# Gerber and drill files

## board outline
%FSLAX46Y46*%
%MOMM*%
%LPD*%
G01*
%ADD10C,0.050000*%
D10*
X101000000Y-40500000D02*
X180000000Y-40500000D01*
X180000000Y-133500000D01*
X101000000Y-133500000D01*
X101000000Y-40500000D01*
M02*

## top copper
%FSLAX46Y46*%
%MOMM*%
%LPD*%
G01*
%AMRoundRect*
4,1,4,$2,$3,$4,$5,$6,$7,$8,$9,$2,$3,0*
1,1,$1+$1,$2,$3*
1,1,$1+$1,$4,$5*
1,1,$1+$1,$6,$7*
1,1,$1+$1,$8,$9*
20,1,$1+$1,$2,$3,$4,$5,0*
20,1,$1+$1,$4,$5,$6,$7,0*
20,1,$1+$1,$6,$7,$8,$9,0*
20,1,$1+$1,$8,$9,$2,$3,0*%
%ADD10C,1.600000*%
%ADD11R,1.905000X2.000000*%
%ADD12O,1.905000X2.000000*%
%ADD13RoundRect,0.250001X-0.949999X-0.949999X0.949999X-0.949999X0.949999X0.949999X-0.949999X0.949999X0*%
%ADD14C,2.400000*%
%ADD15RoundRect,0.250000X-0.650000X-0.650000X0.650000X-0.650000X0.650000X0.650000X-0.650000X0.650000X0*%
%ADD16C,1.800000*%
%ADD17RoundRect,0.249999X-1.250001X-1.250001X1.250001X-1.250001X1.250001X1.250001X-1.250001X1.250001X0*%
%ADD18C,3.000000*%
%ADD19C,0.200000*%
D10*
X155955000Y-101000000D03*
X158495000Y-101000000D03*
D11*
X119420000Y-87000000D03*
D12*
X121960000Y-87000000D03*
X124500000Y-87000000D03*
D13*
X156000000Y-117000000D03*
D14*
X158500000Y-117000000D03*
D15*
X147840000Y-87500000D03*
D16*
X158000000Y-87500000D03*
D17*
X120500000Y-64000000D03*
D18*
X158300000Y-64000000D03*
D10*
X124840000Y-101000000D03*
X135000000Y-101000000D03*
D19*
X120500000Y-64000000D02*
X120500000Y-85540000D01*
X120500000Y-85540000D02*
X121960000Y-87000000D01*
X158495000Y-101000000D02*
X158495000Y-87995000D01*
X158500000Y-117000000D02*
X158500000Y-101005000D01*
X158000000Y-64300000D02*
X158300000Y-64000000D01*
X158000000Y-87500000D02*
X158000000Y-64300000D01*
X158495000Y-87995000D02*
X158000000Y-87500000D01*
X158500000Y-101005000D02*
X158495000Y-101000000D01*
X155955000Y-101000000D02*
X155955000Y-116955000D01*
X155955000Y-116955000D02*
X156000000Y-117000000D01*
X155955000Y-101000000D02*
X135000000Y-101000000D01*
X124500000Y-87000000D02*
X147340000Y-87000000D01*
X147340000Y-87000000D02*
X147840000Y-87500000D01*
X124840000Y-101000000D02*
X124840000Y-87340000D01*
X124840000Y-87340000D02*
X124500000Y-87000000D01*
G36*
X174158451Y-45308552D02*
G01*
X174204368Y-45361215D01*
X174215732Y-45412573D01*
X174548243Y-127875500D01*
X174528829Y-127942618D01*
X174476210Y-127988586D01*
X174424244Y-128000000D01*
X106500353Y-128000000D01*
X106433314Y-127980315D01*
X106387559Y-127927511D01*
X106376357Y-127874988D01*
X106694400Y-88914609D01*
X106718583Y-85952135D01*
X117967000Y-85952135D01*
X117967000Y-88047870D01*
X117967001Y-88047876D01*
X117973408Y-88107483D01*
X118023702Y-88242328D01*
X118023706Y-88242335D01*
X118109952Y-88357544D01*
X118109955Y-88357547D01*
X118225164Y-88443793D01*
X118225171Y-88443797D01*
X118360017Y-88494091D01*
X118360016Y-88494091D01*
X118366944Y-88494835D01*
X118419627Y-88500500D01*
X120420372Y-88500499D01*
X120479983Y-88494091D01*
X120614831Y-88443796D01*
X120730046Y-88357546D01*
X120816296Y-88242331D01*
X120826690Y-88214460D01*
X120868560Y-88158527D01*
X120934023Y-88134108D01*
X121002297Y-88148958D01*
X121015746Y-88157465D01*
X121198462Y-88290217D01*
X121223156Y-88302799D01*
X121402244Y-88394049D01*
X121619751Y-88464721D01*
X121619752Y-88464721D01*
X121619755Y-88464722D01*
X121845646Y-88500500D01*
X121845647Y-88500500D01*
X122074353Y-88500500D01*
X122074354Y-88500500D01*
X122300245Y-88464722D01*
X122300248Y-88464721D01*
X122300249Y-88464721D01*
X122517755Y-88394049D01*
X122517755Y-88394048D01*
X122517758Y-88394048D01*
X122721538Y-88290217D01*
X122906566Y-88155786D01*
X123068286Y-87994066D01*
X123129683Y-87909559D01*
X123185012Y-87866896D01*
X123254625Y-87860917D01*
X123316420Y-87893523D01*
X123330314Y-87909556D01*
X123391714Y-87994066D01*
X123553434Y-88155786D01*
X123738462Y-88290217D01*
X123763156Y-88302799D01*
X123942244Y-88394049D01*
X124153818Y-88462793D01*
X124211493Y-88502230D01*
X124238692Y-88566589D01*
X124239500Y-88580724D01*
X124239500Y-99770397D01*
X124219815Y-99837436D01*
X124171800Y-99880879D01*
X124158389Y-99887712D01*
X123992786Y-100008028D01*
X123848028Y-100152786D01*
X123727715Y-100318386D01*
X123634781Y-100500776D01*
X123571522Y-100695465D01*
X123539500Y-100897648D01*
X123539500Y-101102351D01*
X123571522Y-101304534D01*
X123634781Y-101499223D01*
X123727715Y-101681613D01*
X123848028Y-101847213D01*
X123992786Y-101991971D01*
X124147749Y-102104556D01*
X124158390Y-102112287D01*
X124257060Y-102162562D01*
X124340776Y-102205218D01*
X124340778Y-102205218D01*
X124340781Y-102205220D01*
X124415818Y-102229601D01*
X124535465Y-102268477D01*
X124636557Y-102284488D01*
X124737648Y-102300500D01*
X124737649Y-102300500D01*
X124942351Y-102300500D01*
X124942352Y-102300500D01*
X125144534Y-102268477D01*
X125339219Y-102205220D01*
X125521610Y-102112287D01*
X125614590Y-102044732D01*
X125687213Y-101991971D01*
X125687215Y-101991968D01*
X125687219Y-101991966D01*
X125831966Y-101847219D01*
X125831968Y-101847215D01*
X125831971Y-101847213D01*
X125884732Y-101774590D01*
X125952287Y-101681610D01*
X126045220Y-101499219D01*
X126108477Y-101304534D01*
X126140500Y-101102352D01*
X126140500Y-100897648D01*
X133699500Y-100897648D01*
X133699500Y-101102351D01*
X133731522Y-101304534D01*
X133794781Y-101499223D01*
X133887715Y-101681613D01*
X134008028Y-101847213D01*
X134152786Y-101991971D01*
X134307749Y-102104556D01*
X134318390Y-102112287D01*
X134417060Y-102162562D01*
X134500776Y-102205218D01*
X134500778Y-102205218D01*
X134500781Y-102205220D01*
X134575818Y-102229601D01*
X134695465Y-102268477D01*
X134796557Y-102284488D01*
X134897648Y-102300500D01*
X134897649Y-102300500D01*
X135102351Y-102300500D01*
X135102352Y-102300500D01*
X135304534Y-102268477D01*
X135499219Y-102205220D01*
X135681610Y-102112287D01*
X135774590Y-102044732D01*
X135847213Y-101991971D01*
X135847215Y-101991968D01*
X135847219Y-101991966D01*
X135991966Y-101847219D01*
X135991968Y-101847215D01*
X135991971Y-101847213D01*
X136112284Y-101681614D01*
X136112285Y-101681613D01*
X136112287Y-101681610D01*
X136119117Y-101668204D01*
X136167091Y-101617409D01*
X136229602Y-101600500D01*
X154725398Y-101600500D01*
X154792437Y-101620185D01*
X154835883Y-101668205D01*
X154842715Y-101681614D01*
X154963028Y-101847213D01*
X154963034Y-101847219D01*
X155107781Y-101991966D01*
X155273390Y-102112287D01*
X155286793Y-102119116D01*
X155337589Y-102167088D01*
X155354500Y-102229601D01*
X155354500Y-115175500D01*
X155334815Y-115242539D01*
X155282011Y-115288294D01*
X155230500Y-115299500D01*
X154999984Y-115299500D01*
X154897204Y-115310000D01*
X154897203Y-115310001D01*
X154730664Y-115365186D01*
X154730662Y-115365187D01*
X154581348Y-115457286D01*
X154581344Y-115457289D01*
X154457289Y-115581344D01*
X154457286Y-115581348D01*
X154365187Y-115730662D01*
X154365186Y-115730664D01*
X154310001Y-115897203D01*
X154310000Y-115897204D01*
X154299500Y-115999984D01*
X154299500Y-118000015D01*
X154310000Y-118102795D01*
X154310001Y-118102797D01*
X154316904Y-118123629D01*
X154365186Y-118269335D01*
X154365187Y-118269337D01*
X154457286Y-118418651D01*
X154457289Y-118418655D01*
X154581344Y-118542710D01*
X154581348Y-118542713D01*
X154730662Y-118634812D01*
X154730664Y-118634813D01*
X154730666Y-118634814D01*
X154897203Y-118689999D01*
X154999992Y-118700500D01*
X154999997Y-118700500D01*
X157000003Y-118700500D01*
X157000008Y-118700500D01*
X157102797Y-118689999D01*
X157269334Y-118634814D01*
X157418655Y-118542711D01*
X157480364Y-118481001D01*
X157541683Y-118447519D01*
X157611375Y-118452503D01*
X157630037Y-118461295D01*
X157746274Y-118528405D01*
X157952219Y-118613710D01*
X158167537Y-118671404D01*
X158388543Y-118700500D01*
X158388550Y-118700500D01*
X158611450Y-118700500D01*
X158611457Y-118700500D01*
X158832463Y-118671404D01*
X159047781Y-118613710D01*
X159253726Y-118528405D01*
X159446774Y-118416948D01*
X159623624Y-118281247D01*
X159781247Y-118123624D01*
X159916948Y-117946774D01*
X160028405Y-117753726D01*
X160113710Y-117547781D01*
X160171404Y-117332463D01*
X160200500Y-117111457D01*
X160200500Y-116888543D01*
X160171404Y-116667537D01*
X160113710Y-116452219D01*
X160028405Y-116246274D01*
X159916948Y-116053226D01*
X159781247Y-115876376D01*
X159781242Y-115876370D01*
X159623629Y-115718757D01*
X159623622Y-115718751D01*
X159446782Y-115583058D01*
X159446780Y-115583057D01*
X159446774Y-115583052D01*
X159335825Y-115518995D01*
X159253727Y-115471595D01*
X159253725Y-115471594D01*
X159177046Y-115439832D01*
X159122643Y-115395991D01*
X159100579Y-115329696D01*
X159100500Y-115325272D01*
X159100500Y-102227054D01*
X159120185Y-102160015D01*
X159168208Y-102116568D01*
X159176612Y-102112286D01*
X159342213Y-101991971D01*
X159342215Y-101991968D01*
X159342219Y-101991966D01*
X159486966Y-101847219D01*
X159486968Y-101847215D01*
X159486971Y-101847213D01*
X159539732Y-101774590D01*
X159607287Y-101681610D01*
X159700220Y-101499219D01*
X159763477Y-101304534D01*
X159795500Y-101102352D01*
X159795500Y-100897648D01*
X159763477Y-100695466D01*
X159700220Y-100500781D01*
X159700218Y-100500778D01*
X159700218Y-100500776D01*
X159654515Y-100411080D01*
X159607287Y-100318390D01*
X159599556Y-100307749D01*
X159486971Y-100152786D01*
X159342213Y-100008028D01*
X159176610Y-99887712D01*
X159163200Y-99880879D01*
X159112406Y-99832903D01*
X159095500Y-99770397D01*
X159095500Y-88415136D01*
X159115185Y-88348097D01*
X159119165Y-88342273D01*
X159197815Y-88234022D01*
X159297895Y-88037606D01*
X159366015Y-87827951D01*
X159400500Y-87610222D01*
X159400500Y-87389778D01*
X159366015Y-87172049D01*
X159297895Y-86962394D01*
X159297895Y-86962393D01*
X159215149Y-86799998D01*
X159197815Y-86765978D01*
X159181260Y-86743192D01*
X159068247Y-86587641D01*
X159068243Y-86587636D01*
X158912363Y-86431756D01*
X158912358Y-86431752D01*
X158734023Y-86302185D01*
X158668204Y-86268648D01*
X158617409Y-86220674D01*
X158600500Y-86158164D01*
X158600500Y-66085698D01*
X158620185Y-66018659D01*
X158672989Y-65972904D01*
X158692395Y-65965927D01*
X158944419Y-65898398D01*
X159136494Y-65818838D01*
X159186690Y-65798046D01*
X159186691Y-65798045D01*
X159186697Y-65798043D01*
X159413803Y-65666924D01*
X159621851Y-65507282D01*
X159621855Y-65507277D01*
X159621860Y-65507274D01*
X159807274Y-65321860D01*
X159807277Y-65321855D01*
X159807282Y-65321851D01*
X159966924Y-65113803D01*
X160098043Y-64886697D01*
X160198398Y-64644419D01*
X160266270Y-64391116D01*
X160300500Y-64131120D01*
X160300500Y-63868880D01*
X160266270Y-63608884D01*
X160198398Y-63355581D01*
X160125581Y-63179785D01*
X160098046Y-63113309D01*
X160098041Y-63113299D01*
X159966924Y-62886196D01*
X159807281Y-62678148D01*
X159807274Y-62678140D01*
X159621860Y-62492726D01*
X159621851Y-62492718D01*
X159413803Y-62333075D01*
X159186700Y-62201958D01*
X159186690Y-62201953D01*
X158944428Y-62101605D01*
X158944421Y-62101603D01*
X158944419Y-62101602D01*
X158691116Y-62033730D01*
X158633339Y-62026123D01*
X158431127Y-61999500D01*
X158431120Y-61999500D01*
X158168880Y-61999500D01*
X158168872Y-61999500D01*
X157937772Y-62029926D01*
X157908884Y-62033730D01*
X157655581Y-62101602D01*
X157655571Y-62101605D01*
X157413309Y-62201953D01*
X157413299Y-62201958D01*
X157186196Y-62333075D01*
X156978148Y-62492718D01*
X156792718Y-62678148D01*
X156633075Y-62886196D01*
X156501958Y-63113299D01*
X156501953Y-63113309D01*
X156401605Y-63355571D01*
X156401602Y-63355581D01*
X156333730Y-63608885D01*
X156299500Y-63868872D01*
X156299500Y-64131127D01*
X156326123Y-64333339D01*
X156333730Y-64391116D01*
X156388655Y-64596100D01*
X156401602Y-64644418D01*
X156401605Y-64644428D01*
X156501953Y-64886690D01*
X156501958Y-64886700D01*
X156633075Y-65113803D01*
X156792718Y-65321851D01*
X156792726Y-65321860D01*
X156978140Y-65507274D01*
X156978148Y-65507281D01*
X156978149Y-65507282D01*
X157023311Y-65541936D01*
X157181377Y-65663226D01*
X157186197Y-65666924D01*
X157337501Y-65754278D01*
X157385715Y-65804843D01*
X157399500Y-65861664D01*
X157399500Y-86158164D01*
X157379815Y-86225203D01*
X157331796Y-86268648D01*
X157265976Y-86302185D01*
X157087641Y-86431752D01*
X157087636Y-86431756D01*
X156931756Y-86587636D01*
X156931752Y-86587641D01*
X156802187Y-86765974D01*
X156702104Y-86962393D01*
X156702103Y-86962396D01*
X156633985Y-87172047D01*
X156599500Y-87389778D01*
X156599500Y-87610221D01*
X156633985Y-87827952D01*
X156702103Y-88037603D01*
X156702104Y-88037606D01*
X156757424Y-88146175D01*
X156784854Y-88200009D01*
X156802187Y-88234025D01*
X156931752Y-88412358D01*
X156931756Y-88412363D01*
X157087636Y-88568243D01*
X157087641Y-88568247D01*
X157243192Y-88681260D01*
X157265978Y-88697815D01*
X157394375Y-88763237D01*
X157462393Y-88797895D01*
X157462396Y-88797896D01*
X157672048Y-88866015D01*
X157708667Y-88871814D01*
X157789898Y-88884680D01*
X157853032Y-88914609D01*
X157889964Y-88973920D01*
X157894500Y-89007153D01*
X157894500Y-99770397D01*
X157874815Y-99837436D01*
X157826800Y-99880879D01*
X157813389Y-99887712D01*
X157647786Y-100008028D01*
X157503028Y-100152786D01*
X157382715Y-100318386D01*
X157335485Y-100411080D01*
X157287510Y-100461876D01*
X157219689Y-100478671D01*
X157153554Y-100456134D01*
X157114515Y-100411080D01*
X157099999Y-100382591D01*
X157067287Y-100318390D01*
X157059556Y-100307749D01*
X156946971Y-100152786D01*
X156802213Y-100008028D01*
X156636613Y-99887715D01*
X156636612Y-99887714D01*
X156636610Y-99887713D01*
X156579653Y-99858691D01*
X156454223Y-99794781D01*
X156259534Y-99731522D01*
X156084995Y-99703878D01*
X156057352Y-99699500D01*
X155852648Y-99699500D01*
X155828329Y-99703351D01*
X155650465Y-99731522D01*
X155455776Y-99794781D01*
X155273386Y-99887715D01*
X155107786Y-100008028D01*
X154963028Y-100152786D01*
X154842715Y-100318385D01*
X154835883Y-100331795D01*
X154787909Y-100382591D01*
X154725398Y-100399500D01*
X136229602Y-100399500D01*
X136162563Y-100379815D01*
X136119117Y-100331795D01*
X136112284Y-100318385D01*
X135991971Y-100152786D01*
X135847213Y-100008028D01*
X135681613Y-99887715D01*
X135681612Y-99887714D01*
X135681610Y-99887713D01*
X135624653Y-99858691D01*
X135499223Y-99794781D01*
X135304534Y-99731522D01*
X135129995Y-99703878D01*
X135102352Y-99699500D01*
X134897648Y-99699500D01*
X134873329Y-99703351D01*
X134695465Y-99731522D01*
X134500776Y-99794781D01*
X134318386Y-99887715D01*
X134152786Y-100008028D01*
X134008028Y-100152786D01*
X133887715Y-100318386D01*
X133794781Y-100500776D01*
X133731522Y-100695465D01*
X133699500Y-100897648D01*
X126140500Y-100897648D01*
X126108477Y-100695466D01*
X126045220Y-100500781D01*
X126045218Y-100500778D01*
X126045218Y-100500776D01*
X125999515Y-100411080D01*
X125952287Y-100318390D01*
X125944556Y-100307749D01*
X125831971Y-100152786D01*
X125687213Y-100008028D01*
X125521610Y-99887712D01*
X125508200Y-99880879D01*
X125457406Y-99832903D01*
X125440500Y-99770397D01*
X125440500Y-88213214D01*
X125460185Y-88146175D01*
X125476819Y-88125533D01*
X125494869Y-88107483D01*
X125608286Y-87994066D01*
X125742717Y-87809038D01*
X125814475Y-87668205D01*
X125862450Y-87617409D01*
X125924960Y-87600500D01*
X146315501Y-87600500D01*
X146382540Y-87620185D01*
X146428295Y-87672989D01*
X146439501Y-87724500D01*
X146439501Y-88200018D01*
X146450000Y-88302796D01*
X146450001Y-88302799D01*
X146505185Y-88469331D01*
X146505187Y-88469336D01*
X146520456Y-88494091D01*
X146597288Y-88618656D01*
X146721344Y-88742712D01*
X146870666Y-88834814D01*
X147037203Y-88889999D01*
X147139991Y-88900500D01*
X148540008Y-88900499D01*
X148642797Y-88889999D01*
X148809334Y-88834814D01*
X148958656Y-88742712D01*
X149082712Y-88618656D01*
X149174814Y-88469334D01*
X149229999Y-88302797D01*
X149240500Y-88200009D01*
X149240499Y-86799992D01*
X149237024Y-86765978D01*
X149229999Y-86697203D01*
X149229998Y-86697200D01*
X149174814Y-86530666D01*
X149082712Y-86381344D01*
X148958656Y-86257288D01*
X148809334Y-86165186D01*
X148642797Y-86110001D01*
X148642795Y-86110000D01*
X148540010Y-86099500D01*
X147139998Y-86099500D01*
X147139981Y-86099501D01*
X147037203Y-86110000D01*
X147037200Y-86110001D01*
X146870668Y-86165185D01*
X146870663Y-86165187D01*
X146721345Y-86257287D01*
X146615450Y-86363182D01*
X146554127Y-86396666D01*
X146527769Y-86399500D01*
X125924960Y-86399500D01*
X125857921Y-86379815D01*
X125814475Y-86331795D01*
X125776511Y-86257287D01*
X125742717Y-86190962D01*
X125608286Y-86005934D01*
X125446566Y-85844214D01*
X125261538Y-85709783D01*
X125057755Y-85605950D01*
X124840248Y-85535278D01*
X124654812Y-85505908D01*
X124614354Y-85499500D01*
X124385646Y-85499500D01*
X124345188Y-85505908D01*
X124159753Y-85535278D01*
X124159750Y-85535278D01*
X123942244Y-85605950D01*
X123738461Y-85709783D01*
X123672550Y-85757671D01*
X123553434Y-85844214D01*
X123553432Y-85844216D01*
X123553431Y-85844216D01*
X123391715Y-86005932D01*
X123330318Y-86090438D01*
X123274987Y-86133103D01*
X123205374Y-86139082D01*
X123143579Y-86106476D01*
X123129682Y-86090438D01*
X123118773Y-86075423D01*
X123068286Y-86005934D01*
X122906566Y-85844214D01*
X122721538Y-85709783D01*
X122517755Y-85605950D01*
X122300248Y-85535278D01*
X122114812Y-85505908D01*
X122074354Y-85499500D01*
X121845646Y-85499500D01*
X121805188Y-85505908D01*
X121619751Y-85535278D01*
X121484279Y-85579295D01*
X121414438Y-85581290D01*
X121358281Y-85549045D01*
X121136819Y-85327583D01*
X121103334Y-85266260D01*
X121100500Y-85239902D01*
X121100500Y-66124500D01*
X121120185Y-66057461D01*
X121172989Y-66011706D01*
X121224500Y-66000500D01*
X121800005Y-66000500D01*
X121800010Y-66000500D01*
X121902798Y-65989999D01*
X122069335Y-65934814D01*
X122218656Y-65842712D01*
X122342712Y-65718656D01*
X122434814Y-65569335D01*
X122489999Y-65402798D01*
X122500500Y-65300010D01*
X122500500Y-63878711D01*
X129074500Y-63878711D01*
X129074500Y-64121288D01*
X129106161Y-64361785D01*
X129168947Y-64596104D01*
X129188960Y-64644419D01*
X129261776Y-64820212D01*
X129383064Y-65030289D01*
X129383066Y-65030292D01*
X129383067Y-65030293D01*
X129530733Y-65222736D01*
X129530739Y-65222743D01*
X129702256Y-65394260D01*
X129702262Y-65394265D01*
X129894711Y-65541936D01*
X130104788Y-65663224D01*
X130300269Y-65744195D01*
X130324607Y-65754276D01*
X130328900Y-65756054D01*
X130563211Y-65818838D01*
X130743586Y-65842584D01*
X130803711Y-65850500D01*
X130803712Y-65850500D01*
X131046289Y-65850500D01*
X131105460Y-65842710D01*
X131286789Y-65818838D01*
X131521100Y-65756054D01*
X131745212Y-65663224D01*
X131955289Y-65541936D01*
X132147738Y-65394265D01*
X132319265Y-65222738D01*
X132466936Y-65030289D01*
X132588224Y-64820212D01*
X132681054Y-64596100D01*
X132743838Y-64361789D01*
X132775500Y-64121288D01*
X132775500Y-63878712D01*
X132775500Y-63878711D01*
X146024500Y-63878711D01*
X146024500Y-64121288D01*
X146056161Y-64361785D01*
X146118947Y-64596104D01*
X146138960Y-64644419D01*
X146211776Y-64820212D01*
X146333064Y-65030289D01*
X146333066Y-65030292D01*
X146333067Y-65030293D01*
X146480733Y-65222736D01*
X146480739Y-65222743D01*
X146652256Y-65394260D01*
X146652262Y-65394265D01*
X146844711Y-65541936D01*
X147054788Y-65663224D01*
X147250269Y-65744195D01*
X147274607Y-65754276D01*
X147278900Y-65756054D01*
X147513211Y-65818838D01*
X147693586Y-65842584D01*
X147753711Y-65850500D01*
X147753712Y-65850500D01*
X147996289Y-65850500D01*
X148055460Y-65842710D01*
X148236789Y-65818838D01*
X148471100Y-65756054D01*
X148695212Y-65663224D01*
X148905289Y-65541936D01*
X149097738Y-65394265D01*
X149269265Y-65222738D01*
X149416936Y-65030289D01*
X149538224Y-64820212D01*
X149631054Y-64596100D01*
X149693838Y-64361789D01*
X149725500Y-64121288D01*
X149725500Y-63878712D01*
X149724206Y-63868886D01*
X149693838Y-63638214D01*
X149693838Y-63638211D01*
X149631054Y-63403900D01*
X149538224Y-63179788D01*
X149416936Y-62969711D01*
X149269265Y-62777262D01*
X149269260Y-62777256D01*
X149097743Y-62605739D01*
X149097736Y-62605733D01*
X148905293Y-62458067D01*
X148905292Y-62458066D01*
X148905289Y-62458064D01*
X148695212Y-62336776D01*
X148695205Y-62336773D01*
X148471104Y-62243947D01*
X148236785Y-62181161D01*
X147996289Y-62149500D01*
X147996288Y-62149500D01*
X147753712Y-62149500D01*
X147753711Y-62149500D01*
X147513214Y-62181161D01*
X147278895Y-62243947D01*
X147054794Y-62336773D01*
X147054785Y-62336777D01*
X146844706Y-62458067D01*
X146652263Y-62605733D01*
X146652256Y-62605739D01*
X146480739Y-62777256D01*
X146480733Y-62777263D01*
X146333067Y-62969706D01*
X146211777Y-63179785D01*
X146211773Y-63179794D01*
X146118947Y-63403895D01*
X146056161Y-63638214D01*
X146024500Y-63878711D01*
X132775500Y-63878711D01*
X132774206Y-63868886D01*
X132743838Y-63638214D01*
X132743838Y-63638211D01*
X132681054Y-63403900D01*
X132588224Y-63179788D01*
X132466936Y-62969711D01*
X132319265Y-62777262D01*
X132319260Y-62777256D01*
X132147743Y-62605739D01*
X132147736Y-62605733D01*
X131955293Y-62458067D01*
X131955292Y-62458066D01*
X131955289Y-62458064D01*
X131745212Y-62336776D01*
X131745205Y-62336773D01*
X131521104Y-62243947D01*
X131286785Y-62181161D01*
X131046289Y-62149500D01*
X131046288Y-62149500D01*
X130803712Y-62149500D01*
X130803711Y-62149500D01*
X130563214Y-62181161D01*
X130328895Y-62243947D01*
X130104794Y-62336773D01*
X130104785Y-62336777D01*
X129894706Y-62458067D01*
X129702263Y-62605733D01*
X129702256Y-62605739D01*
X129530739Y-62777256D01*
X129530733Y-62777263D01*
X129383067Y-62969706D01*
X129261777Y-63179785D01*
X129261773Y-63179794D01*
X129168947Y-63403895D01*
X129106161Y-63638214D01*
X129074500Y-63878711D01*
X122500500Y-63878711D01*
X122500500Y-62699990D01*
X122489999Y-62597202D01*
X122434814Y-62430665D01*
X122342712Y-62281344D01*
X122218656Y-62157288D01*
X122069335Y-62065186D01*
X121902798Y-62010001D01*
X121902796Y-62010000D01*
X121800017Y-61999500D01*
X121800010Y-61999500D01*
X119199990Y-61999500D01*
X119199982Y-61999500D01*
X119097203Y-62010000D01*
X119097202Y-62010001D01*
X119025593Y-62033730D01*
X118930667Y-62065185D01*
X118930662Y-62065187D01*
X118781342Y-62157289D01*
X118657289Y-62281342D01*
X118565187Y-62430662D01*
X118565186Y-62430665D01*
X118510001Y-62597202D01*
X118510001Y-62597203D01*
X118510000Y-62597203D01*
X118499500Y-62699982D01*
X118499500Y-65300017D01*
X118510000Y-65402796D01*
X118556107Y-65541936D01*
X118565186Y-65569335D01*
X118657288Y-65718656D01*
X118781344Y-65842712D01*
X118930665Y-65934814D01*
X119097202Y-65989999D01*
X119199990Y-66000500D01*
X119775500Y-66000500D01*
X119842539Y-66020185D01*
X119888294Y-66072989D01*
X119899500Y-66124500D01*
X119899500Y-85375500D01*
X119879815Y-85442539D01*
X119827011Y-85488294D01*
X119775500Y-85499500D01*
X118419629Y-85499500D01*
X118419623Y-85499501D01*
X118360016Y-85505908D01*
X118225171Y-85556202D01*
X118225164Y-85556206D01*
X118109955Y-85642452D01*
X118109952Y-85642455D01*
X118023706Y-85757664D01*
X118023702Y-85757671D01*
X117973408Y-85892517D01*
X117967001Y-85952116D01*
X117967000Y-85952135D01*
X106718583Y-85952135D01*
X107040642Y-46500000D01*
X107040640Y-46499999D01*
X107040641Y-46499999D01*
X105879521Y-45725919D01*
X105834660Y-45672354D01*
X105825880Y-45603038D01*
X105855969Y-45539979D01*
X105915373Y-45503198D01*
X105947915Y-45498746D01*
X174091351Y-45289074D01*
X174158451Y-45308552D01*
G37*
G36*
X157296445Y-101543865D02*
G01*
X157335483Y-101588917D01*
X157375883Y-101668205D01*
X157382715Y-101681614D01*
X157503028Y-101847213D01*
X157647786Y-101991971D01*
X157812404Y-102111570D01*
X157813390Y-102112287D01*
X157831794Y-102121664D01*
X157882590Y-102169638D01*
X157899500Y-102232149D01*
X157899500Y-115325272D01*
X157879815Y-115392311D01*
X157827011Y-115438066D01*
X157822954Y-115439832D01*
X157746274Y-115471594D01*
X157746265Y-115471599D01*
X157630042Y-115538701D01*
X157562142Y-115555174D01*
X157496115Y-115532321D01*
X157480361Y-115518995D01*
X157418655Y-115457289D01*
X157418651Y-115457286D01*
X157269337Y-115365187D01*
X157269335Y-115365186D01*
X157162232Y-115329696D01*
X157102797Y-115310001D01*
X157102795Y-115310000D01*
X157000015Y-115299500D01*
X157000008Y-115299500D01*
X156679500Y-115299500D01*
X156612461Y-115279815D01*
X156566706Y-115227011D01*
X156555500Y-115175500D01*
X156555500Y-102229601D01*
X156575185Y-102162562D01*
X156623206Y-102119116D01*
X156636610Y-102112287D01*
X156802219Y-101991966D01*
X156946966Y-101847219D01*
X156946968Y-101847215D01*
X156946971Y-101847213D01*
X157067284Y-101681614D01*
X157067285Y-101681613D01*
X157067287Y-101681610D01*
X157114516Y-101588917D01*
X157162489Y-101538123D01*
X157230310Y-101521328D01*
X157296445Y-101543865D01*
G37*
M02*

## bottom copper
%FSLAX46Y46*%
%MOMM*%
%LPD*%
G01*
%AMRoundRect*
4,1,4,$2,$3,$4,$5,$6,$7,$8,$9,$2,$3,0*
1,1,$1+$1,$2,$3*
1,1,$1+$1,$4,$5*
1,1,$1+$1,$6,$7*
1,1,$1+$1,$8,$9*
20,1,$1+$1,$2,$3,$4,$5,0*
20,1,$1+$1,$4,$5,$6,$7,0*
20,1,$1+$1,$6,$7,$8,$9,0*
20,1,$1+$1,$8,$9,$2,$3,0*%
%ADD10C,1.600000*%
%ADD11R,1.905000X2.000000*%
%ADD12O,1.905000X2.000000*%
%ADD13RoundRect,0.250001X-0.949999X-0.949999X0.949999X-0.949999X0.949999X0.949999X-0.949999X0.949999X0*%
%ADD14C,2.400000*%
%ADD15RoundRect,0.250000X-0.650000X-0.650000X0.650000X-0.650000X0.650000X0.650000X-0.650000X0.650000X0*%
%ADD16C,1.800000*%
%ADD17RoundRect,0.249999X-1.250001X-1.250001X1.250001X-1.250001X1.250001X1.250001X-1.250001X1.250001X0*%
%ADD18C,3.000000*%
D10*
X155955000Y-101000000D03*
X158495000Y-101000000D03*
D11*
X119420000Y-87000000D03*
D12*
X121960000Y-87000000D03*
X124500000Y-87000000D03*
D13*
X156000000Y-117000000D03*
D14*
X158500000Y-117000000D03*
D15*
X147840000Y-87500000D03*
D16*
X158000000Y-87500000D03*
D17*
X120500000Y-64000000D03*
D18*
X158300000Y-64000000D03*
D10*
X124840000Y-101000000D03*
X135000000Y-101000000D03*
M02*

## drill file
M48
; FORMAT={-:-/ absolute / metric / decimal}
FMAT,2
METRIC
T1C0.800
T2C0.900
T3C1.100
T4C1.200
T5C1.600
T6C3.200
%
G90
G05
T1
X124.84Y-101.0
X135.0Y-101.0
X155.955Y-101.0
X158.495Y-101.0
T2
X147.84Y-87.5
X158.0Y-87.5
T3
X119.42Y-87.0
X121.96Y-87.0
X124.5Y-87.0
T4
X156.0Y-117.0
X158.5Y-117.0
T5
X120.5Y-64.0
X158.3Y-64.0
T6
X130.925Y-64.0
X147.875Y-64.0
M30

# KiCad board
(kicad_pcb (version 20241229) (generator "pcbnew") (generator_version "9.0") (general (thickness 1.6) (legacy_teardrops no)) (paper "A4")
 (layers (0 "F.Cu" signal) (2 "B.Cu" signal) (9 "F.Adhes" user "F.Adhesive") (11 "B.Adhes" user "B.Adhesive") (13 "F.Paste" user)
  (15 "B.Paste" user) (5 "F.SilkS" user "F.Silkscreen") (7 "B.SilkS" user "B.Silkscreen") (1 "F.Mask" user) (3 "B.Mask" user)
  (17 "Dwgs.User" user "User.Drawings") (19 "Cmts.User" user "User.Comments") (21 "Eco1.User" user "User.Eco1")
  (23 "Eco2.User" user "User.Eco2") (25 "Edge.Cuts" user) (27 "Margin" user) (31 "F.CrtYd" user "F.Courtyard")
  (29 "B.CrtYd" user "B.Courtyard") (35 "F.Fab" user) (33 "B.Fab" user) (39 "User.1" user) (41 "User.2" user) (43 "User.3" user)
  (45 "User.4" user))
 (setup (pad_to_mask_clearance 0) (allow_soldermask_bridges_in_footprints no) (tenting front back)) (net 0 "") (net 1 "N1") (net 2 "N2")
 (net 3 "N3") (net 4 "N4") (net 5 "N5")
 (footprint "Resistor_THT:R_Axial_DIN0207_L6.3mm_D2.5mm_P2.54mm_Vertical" (layer "F.Cu") (at 155.955 101)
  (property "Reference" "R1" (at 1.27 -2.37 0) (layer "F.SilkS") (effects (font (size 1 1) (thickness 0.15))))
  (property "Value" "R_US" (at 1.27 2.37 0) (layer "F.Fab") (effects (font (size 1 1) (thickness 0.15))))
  (pad "1" thru_hole circle (at 0 0) (size 1.6 1.6) (drill 0.8) (layers "*.Cu" "*.Mask") (remove_unused_layers no) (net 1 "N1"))
  (pad "2" thru_hole circle (at 2.54 0) (size 1.6 1.6) (drill 0.8) (layers "*.Cu" "*.Mask") (remove_unused_layers no) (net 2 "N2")))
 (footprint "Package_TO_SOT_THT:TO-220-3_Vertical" (layer "F.Cu") (at 119.42 87)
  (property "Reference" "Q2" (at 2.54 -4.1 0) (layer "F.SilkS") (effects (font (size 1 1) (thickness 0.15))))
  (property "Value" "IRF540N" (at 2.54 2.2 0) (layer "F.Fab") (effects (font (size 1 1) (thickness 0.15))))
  (pad "1" thru_hole rect (at 0 0) (size 1.905 2) (drill 1.1) (layers "*.Cu" "*.Mask") (remove_unused_layers no) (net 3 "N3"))
  (pad "2" thru_hole oval (at 2.54 0) (size 1.905 2) (drill 1.1) (layers "*.Cu" "*.Mask") (remove_unused_layers no) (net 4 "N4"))
  (pad "3" thru_hole oval (at 5.08 0) (size 1.905 2) (drill 1.1) (layers "*.Cu" "*.Mask") (remove_unused_layers no) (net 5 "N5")))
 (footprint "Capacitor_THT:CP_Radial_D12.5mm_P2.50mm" (layer "F.Cu") (at 156 117)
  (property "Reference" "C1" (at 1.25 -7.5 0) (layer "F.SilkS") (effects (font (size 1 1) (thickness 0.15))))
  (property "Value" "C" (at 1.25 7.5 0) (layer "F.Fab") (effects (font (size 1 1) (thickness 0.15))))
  (pad "1" thru_hole roundrect (at 0 0) (size 2.4 2.4) (drill 1.2) (layers "*.Cu" "*.Mask") (remove_unused_layers no)
   (roundrect_rratio 0.104167) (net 1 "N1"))
  (pad "2" thru_hole circle (at 2.5 0) (size 2.4 2.4) (drill 1.2) (layers "*.Cu" "*.Mask") (remove_unused_layers no) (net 2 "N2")))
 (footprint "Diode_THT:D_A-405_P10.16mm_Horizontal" (layer "F.Cu") (at 147.84 87.5)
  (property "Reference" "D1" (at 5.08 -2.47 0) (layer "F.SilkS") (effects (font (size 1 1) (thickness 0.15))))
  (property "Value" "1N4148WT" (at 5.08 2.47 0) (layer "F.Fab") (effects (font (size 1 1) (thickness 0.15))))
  (pad "1" thru_hole roundrect (at 0 0) (size 1.8 1.8) (drill 0.9) (layers "*.Cu" "*.Mask") (remove_unused_layers no)
   (roundrect_rratio 0.138889) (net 5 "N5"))
  (pad "2" thru_hole circle (at 10.16 0) (size 1.8 1.8) (drill 0.9) (layers "*.Cu" "*.Mask") (remove_unused_layers no) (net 2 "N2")))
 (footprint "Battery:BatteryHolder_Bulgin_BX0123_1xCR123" (layer "F.Cu") (at 120.5 64)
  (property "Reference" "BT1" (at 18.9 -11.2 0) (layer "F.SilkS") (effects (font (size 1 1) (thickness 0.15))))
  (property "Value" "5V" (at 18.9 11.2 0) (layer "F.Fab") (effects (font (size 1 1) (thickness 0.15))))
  (pad "" np_thru_hole circle (at 10.425 0) (size 3.2 3.2) (drill 3.2) (layers "*.Cu" "*.Mask"))
  (pad "" np_thru_hole circle (at 27.375 0) (size 3.2 3.2) (drill 3.2) (layers "*.Cu" "*.Mask"))
  (pad "1" thru_hole roundrect (at 0 0) (size 3 3) (drill 1.6) (layers "*.Cu" "*.Mask") (remove_unused_layers no)
   (roundrect_rratio 0.083333) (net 4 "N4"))
  (pad "2" thru_hole circle (at 37.8 0) (size 3 3) (drill 1.6) (layers "*.Cu" "*.Mask") (remove_unused_layers no) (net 2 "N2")))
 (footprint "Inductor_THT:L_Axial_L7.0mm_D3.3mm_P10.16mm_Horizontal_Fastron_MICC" (layer "F.Cu") (at 124.84 101)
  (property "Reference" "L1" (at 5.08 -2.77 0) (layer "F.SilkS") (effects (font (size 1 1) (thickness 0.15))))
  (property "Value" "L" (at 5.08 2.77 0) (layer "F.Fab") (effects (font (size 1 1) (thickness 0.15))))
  (pad "1" thru_hole circle (at 0 0) (size 1.6 1.6) (drill 0.8) (layers "*.Cu" "*.Mask") (remove_unused_layers no) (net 5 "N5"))
  (pad "2" thru_hole circle (at 10.16 0) (size 1.6 1.6) (drill 0.8) (layers "*.Cu" "*.Mask") (remove_unused_layers no) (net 1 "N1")))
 (gr_rect (start 101 40.5) (end 180 133.5) (stroke (width 0.05) (type default)) (fill no) (layer "Edge.Cuts"))
 (segment (start 120.5 64) (end 120.5 85.54) (width 0.2) (layer "F.Cu") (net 4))
 (segment (start 120.5 85.54) (end 121.96 87) (width 0.2) (layer "F.Cu") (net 4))
 (segment (start 158.495 101) (end 158.495 87.995) (width 0.2) (layer "F.Cu") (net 2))
 (segment (start 158.5 117) (end 158.5 101.005) (width 0.2) (layer "F.Cu") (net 2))
 (segment (start 158 64.3) (end 158.3 64) (width 0.2) (layer "F.Cu") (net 2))
 (segment (start 158 87.5) (end 158 64.3) (width 0.2) (layer "F.Cu") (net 2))
 (segment (start 158.495 87.995) (end 158 87.5) (width 0.2) (layer "F.Cu") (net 2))
 (segment (start 158.5 101.005) (end 158.495 101) (width 0.2) (layer "F.Cu") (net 2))
 (segment (start 155.955 101) (end 155.955 116.955) (width 0.2) (layer "F.Cu") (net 1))
 (segment (start 155.955 116.955) (end 156 117) (width 0.2) (layer "F.Cu") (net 1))
 (segment (start 155.955 101) (end 135 101) (width 0.2) (layer "F.Cu") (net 1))
 (segment (start 124.5 87) (end 147.34 87) (width 0.2) (layer "F.Cu") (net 5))
 (segment (start 147.34 87) (end 147.84 87.5) (width 0.2) (layer "F.Cu") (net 5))
 (segment (start 124.84 101) (end 124.84 87.34) (width 0.2) (layer "F.Cu") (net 5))
 (segment (start 124.84 87.34) (end 124.5 87) (width 0.2) (layer "F.Cu") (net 5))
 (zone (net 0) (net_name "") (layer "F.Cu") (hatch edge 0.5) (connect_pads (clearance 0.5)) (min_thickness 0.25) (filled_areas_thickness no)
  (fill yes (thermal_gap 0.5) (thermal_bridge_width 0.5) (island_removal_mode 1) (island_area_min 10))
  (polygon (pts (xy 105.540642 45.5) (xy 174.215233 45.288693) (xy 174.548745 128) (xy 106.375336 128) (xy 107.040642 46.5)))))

